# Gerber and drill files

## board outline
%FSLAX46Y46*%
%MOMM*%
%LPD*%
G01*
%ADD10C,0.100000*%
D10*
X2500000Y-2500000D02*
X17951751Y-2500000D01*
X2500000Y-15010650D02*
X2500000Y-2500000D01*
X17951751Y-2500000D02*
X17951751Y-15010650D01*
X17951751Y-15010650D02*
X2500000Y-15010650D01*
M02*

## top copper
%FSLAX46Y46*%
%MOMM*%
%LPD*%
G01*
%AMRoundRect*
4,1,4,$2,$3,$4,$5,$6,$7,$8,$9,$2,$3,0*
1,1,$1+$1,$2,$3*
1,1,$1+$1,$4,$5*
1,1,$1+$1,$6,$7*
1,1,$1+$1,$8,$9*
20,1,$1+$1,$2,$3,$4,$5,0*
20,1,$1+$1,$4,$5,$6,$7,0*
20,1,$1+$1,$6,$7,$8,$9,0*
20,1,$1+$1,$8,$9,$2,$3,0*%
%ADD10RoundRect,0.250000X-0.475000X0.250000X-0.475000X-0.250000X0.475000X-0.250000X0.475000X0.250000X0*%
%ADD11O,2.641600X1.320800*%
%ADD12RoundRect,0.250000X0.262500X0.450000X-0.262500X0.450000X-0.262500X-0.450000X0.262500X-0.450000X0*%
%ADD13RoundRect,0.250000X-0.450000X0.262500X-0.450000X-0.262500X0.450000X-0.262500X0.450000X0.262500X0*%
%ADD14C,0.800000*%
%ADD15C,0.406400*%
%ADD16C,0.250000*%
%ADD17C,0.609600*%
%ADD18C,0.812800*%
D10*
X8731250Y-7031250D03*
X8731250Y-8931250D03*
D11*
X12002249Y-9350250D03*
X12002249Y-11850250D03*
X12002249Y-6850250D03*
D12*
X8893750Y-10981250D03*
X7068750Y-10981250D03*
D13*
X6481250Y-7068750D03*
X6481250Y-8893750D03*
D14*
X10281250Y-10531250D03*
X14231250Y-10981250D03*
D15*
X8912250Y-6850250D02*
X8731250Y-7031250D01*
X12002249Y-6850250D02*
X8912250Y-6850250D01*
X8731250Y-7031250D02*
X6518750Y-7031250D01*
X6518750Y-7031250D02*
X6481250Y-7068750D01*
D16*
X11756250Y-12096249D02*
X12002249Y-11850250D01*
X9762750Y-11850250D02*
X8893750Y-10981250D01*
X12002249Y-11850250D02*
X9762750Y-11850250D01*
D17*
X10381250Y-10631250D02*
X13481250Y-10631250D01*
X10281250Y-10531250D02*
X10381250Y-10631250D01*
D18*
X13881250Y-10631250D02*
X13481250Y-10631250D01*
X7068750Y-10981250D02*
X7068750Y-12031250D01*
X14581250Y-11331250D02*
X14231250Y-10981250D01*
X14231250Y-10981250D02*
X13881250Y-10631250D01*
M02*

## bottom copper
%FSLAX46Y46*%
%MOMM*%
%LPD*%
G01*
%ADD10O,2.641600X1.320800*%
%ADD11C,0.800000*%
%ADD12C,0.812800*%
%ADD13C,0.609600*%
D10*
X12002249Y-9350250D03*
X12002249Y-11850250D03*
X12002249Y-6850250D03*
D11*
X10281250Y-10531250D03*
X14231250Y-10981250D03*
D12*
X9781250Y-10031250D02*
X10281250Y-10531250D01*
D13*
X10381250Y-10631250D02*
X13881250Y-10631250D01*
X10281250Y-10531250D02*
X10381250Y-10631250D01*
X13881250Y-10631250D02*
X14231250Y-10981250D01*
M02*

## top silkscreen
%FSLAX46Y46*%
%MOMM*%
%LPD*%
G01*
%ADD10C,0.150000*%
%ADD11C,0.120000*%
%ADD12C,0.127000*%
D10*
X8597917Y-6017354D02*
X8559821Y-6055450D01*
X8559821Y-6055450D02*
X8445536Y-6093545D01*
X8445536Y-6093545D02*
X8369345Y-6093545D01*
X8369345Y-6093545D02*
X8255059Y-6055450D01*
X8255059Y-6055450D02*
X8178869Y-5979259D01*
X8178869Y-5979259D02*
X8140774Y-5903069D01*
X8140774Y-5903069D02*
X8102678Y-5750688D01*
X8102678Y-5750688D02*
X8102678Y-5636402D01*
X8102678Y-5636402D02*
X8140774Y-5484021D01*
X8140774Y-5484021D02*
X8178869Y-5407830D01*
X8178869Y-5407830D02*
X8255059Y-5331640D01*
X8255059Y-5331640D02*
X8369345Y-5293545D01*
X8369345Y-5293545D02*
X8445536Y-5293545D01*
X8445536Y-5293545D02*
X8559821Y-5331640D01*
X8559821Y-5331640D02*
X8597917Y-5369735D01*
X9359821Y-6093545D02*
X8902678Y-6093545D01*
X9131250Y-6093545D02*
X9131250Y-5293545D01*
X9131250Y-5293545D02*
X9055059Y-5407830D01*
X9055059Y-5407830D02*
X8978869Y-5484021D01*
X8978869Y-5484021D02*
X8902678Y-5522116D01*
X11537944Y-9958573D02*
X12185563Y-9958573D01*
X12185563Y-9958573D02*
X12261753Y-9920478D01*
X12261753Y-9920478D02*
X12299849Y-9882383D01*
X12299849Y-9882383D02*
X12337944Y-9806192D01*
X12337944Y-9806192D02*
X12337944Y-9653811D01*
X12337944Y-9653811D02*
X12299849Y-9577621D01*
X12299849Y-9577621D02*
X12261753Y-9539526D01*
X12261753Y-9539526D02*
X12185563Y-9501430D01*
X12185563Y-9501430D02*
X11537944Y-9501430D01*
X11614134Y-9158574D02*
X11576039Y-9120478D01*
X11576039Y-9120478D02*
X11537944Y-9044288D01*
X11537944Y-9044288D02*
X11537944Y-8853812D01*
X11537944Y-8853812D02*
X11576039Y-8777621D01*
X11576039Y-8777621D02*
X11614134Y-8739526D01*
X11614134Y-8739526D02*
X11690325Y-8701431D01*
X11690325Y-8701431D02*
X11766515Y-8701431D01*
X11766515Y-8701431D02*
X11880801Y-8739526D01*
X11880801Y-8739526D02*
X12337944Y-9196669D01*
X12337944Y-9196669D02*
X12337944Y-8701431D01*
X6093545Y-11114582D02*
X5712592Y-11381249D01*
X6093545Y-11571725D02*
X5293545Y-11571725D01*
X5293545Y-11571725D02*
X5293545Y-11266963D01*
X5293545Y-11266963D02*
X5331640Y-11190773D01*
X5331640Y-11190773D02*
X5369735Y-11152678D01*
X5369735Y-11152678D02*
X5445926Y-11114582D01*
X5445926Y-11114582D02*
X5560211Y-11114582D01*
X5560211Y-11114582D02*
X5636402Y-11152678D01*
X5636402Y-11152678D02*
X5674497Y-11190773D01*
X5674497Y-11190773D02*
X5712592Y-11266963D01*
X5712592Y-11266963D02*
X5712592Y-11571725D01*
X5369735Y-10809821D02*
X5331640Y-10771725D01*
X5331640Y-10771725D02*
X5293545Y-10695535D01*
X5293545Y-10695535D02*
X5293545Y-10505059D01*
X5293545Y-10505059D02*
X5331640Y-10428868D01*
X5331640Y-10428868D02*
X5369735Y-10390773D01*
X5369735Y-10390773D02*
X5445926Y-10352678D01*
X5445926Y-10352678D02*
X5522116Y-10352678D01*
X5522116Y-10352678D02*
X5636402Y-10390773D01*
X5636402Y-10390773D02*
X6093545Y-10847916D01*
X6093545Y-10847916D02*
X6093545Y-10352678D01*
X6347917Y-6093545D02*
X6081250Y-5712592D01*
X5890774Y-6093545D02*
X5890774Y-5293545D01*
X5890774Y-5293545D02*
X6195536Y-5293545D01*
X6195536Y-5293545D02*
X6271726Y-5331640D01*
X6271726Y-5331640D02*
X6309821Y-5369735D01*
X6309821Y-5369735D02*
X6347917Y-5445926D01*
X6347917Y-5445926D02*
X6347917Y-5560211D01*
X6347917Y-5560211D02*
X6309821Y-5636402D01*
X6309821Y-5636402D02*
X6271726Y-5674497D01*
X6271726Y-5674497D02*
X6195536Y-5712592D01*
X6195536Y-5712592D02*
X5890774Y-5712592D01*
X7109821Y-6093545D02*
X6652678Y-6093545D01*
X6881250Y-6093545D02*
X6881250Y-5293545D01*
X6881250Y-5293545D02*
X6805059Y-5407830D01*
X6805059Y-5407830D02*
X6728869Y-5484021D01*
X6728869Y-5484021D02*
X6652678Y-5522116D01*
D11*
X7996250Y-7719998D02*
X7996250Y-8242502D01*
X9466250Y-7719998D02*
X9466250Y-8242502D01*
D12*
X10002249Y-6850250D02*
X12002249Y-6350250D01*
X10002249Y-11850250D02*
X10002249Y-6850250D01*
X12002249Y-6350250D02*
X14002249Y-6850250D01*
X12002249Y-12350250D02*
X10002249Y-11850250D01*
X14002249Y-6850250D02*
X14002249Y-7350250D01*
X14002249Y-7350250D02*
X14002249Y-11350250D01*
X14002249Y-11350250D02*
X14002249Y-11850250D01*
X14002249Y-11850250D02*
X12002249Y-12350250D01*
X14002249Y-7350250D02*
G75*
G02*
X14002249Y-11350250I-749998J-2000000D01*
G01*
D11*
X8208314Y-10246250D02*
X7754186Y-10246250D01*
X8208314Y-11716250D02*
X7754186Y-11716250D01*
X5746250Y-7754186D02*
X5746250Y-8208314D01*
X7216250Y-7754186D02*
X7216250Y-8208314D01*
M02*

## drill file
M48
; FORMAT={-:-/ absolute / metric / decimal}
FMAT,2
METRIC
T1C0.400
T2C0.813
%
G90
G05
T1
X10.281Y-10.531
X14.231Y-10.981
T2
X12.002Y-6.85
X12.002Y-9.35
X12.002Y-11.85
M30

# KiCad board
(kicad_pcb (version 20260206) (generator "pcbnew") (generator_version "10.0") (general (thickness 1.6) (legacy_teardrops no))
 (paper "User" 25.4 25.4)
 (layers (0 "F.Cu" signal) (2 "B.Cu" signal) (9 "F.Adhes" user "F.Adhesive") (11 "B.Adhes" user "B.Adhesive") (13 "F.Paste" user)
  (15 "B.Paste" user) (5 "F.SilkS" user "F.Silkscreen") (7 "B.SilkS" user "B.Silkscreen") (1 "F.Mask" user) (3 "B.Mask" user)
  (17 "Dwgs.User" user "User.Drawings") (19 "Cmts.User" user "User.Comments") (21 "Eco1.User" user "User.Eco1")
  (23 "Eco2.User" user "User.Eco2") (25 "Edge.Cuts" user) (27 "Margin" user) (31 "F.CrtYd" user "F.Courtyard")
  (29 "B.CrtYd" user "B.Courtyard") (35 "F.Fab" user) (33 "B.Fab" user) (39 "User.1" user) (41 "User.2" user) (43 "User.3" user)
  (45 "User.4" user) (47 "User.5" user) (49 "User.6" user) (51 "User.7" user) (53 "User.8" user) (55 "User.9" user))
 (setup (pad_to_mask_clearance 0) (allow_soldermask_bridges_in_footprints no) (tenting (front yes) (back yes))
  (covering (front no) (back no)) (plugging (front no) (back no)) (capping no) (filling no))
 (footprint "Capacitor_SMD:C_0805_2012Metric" (layer "F.Cu") (at 8.73125 7.98125 -90)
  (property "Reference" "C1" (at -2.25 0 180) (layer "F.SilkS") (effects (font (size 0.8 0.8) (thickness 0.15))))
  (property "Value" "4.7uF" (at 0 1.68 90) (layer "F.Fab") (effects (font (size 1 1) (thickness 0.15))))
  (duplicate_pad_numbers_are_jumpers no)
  (fp_line (start -0.261252 0.735) (end 0.261252 0.735) (stroke (width 0.12) (type solid)) (layer "F.SilkS"))
  (fp_line (start -0.261252 -0.735) (end 0.261252 -0.735) (stroke (width 0.12) (type solid)) (layer "F.SilkS"))
  (pad "1" smd roundrect (at -0.95 0 270) (size 1 1.45) (layers "F.Cu" "F.Mask" "F.Paste") (roundrect_rratio 0.25) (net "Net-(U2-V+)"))
  (pad "2" smd roundrect (at 0.95 0 270) (size 1 1.45) (layers "F.Cu" "F.Mask" "F.Paste") (roundrect_rratio 0.25) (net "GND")))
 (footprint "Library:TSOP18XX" (layer "F.Cu") (at 11.975649 9.34905 90)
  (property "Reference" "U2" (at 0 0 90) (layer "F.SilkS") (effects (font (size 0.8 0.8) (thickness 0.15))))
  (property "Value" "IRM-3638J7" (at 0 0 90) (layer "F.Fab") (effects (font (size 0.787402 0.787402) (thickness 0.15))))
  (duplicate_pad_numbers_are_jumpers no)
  (fp_line (start 2.4988 -1.9734) (end 2.9988 0.0266) (stroke (width 0.127) (type solid)) (layer "F.SilkS"))
  (fp_line (start -2.5012 -1.9734) (end 2.4988 -1.9734) (stroke (width 0.127) (type solid)) (layer "F.SilkS"))
  (fp_line (start 2.9988 0.0266) (end 2.4988 2.0266) (stroke (width 0.127) (type solid)) (layer "F.SilkS"))
  (fp_line (start -3.0012 0.0266) (end -2.5012 -1.9734) (stroke (width 0.127) (type solid)) (layer "F.SilkS"))
  (fp_line (start 2.4988 2.0266) (end 1.9988 2.0266) (stroke (width 0.127) (type solid)) (layer "F.SilkS"))
  (fp_line (start 1.9988 2.0266) (end -2.0012 2.0266) (stroke (width 0.127) (type solid)) (layer "F.SilkS"))
  (fp_line (start -2.0012 2.0266) (end -2.5012 2.0266) (stroke (width 0.127) (type solid)) (layer "F.SilkS"))
  (fp_line (start -2.5012 2.0266) (end -3.0012 0.0266) (stroke (width 0.127) (type solid)) (layer "F.SilkS"))
  (fp_arc (start 1.9988 2.0266) (mid -0.0012 3.412602) (end -2.0012 2.0266) (stroke (width 0.127) (type solid)) (layer "F.SilkS"))
  (pad "GND" thru_hole oval (at -0.0012 0.0266 90) (size 1.3208 2.6416) (drill 0.8128) (layers "*.Cu" "*.Mask") (remove_unused_layers no)
   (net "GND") (solder_mask_margin 0.102))
  (pad "OUT" thru_hole oval (at -2.5012 0.0266 90) (size 1.3208 2.6416) (drill 0.8128) (layers "*.Cu" "*.Mask") (remove_unused_layers no)
   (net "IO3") (solder_mask_margin 0.102))
  (pad "VCC" thru_hole oval (at 2.4988 0.0266 90) (size 1.3208 2.6416) (drill 0.8128) (layers "*.Cu" "*.Mask") (remove_unused_layers no)
   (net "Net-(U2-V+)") (solder_mask_margin 0.102)))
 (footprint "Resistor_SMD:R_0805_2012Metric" (layer "F.Cu") (at 7.98125 10.98125 180)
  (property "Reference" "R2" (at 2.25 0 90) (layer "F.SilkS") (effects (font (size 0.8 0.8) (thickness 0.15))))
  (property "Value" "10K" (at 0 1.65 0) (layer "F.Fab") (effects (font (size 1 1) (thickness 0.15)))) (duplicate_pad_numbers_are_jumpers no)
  (fp_line (start -0.227064 0.735) (end 0.227064 0.735) (stroke (width 0.12) (type solid)) (layer "F.SilkS"))
  (fp_line (start -0.227064 -0.735) (end 0.227064 -0.735) (stroke (width 0.12) (type solid)) (layer "F.SilkS"))
  (pad "1" smd roundrect (at -0.9125 0 180) (size 1.025 1.4) (layers "F.Cu" "F.Mask" "F.Paste") (roundrect_rratio 0.243902439) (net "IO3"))
  (pad "2" smd roundrect (at 0.9125 0 180) (size 1.025 1.4) (layers "F.Cu" "F.Mask" "F.Paste") (roundrect_rratio 0.243902439) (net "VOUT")))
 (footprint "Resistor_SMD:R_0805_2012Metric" (layer "F.Cu") (at 6.48125 7.98125 -90)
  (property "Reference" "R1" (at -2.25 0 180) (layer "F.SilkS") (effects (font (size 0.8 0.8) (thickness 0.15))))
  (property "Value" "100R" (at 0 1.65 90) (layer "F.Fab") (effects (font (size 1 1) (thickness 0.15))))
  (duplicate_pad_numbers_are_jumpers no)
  (fp_line (start -0.227064 0.735) (end 0.227064 0.735) (stroke (width 0.12) (type solid)) (layer "F.SilkS"))
  (fp_line (start -0.227064 -0.735) (end 0.227064 -0.735) (stroke (width 0.12) (type solid)) (layer "F.SilkS"))
  (pad "1" smd roundrect (at -0.9125 0 270) (size 1.025 1.4) (layers "F.Cu" "F.Mask" "F.Paste") (roundrect_rratio 0.243902439)
   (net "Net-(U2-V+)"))
  (pad "2" smd roundrect (at 0.9125 0 270) (size 1.025 1.4) (layers "F.Cu" "F.Mask" "F.Paste") (roundrect_rratio 0.243902439) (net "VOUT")))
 (gr_line (start 2.5 2.5) (end 17.951751 2.5) (stroke (width 0.1) (type default)) (layer "Edge.Cuts"))
 (gr_line (start 2.5 15.01065) (end 2.5 2.5) (stroke (width 0.1) (type default)) (layer "Edge.Cuts"))
 (gr_line (start 17.951751 2.5) (end 17.951751 15.01065) (stroke (width 0.1) (type default)) (layer "Edge.Cuts"))
 (gr_line (start 17.951751 15.01065) (end 2.5 15.01065) (stroke (width 0.1) (type default)) (layer "Edge.Cuts"))
 (segment (start 8.91225 6.85025) (end 8.73125 7.03125) (width 0.4064) (layer "F.Cu") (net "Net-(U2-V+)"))
 (segment (start 12.002249 6.85025) (end 8.91225 6.85025) (width 0.4064) (layer "F.Cu") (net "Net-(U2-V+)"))
 (segment (start 8.73125 7.03125) (end 6.51875 7.03125) (width 0.4064) (layer "F.Cu") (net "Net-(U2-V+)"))
 (segment (start 6.51875 7.03125) (end 6.48125 7.06875) (width 0.4064) (layer "F.Cu") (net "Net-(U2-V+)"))
 (segment (start 11.75625 12.096249) (end 12.002249 11.85025) (width 0.25) (layer "F.Cu") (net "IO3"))
 (segment (start 9.76275 11.85025) (end 8.89375 10.98125) (width 0.25) (layer "F.Cu") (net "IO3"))
 (segment (start 12.002249 11.85025) (end 9.76275 11.85025) (width 0.25) (layer "F.Cu") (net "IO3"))
 (segment (start 10.38125 10.63125) (end 13.48125 10.63125) (width 0.6096) (layer "F.Cu") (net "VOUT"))
 (segment (start 10.28125 10.53125) (end 10.38125 10.63125) (width 0.6096) (layer "F.Cu") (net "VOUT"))
 (segment (start 13.88125 10.63125) (end 13.48125 10.63125) (width 0.8128) (layer "F.Cu") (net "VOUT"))
 (segment (start 7.06875 10.98125) (end 7.06875 12.03125) (width 0.8128) (layer "F.Cu") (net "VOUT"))
 (segment (start 14.58125 11.33125) (end 14.23125 10.98125) (width 0.8128) (layer "F.Cu") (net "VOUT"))
 (segment (start 14.23125 10.98125) (end 13.88125 10.63125) (width 0.8128) (layer "F.Cu") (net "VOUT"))
 (via (at 10.28125 10.53125) (size 0.8) (drill 0.4) (layers "F.Cu" "B.Cu") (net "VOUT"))
 (via (at 14.23125 10.98125) (size 0.8) (drill 0.4) (layers "F.Cu" "B.Cu") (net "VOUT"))
 (segment (start 9.78125 10.03125) (end 10.28125 10.53125) (width 0.8128) (layer "B.Cu") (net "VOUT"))
 (segment (start 10.38125 10.63125) (end 13.88125 10.63125) (width 0.6096) (layer "B.Cu") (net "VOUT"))
 (segment (start 10.28125 10.53125) (end 10.38125 10.63125) (width 0.6096) (layer "B.Cu") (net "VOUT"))
 (segment (start 13.88125 10.63125) (end 14.23125 10.98125) (width 0.6096) (layer "B.Cu") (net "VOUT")))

